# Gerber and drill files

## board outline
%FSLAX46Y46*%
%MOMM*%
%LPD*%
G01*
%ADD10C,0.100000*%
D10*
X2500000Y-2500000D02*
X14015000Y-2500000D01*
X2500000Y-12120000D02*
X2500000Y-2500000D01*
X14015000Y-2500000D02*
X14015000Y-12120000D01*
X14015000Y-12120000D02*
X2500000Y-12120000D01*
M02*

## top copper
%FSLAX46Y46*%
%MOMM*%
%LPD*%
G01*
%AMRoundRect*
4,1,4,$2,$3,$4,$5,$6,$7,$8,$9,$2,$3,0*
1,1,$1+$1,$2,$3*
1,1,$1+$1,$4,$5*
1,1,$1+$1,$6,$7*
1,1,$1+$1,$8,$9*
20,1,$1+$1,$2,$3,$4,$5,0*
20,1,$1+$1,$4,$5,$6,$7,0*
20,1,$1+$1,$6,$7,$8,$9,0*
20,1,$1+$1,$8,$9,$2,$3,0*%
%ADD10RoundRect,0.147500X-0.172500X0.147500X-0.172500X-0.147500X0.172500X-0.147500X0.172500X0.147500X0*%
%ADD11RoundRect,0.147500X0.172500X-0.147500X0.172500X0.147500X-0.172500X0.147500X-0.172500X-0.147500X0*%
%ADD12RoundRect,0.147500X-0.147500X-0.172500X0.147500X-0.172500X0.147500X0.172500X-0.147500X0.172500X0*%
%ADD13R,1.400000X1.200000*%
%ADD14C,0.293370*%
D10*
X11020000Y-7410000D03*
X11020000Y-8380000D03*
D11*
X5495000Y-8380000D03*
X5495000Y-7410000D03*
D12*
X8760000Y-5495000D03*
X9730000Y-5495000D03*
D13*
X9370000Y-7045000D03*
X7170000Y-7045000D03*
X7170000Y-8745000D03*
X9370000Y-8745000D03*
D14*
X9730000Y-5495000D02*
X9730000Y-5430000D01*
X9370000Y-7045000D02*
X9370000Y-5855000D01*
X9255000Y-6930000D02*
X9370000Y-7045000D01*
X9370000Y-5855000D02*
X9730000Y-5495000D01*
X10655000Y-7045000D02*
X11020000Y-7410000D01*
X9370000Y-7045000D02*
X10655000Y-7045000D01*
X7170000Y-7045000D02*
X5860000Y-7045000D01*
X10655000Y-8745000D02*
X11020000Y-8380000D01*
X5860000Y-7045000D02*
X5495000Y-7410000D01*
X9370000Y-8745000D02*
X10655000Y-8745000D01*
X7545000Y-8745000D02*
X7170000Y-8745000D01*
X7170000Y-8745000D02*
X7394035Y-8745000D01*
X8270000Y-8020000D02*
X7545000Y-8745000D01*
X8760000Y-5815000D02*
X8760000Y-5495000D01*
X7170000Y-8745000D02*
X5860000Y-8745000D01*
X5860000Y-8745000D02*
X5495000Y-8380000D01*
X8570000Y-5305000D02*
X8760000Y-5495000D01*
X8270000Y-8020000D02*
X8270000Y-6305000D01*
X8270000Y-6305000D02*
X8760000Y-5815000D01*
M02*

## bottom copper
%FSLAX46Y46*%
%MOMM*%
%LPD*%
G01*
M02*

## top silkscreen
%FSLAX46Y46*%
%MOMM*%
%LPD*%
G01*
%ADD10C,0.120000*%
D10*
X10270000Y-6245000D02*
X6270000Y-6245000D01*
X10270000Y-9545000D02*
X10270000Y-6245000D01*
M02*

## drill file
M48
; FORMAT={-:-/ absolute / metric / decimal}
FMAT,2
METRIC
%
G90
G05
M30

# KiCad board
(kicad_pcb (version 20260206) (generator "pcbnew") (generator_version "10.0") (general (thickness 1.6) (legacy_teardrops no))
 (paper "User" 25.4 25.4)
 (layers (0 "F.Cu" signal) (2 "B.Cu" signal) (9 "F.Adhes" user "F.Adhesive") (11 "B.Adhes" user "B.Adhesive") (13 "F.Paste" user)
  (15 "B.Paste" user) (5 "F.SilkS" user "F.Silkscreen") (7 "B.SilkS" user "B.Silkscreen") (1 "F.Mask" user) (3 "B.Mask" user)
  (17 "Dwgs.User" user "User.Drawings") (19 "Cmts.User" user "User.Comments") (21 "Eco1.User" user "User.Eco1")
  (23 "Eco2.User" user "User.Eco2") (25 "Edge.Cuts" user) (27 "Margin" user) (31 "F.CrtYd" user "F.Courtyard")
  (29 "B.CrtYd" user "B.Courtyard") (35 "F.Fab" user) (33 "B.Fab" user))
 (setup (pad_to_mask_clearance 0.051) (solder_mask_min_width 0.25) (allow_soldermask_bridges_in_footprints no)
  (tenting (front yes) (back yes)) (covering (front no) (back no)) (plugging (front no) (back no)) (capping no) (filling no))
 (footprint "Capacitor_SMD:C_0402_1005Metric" (layer "F.Cu") (at 11.02 7.895 -90)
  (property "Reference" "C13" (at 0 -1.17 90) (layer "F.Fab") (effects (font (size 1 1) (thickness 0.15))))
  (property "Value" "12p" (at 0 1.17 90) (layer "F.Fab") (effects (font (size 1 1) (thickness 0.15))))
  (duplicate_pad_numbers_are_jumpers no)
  (pad "1" smd roundrect (at -0.485 0 270) (size 0.59 0.64) (layers "F.Cu" "F.Mask" "F.Paste") (roundrect_rratio 0.25) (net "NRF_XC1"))
  (pad "2" smd roundrect (at 0.485 0 270) (size 0.59 0.64) (layers "F.Cu" "F.Mask" "F.Paste") (roundrect_rratio 0.25) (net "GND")))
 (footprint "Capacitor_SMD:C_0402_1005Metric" (layer "F.Cu") (at 5.495 7.895 90)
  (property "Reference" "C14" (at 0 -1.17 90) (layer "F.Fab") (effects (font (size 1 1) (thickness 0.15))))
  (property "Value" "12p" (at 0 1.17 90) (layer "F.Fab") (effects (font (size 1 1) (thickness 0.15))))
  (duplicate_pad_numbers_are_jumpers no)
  (pad "1" smd roundrect (at -0.485 0 90) (size 0.59 0.64) (layers "F.Cu" "F.Mask" "F.Paste") (roundrect_rratio 0.25) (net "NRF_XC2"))
  (pad "2" smd roundrect (at 0.485 0 90) (size 0.59 0.64) (layers "F.Cu" "F.Mask" "F.Paste") (roundrect_rratio 0.25) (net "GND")))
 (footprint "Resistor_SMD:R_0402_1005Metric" (layer "F.Cu") (at 9.245 5.495)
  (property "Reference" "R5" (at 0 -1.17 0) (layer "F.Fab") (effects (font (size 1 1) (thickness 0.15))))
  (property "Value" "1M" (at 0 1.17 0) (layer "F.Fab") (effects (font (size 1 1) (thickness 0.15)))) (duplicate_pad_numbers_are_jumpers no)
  (pad "1" smd roundrect (at -0.485 0) (size 0.59 0.64) (layers "F.Cu" "F.Mask" "F.Paste") (roundrect_rratio 0.25) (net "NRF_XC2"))
  (pad "2" smd roundrect (at 0.485 0) (size 0.59 0.64) (layers "F.Cu" "F.Mask" "F.Paste") (roundrect_rratio 0.25) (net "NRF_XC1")))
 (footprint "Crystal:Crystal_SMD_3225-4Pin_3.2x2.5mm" (layer "F.Cu") (at 8.27 7.895 180)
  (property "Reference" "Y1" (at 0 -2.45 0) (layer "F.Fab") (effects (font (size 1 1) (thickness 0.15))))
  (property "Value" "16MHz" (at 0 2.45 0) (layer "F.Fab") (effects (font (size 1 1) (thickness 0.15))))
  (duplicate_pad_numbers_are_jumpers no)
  (fp_line (start -2 1.65) (end 2 1.65) (stroke (width 0.12) (type solid)) (layer "F.SilkS"))
  (fp_line (start -2 -1.65) (end -2 1.65) (stroke (width 0.12) (type solid)) (layer "F.SilkS"))
  (pad "1" smd rect (at -1.1 0.85 180) (size 1.4 1.2) (layers "F.Cu" "F.Mask" "F.Paste") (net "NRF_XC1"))
  (pad "2" smd rect (at 1.1 0.85 180) (size 1.4 1.2) (layers "F.Cu" "F.Mask" "F.Paste") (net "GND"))
  (pad "3" smd rect (at 1.1 -0.85 180) (size 1.4 1.2) (layers "F.Cu" "F.Mask" "F.Paste") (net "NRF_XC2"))
  (pad "4" smd rect (at -1.1 -0.85 180) (size 1.4 1.2) (layers "F.Cu" "F.Mask" "F.Paste") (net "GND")))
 (gr_line (start 2.5 2.5) (end 14.015 2.5) (stroke (width 0.1) (type default)) (layer "Edge.Cuts"))
 (gr_line (start 2.5 12.12) (end 2.5 2.5) (stroke (width 0.1) (type default)) (layer "Edge.Cuts"))
 (gr_line (start 14.015 2.5) (end 14.015 12.12) (stroke (width 0.1) (type default)) (layer "Edge.Cuts"))
 (gr_line (start 14.015 12.12) (end 2.5 12.12) (stroke (width 0.1) (type default)) (layer "Edge.Cuts"))
 (segment (start 9.73 5.495) (end 9.73 5.43) (width 0.29337) (layer "F.Cu") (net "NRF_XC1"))
 (segment (start 9.37 7.045) (end 9.37 5.855) (width 0.29337) (layer "F.Cu") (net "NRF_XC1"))
 (segment (start 9.255 6.93) (end 9.37 7.045) (width 0.29337) (layer "F.Cu") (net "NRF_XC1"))
 (segment (start 9.37 5.855) (end 9.73 5.495) (width 0.29337) (layer "F.Cu") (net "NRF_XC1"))
 (segment (start 10.655 7.045) (end 11.02 7.41) (width 0.29337) (layer "F.Cu") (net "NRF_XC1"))
 (segment (start 9.37 7.045) (end 10.655 7.045) (width 0.29337) (layer "F.Cu") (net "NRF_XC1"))
 (segment (start 7.17 7.045) (end 5.86 7.045) (width 0.29337) (layer "F.Cu") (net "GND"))
 (segment (start 10.655 8.745) (end 11.02 8.38) (width 0.29337) (layer "F.Cu") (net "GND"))
 (segment (start 5.86 7.045) (end 5.495 7.41) (width 0.29337) (layer "F.Cu") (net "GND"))
 (segment (start 9.37 8.745) (end 10.655 8.745) (width 0.29337) (layer "F.Cu") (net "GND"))
 (segment (start 7.545 8.745) (end 7.17 8.745) (width 0.29337) (layer "F.Cu") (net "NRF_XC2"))
 (segment (start 7.17 8.745) (end 7.394035 8.745) (width 0.29337) (layer "F.Cu") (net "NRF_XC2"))
 (segment (start 8.27 8.02) (end 7.545 8.745) (width 0.29337) (layer "F.Cu") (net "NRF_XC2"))
 (segment (start 8.76 5.815) (end 8.76 5.495) (width 0.29337) (layer "F.Cu") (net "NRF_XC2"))
 (segment (start 7.17 8.745) (end 5.86 8.745) (width 0.29337) (layer "F.Cu") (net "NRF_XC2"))
 (segment (start 5.86 8.745) (end 5.495 8.38) (width 0.29337) (layer "F.Cu") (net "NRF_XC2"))
 (segment (start 8.57 5.305) (end 8.76 5.495) (width 0.29337) (layer "F.Cu") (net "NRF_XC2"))
 (segment (start 8.27 8.02) (end 8.27 6.305) (width 0.29337) (layer "F.Cu") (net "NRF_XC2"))
 (segment (start 8.27 6.305) (end 8.76 5.815) (width 0.29337) (layer "F.Cu") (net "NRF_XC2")))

